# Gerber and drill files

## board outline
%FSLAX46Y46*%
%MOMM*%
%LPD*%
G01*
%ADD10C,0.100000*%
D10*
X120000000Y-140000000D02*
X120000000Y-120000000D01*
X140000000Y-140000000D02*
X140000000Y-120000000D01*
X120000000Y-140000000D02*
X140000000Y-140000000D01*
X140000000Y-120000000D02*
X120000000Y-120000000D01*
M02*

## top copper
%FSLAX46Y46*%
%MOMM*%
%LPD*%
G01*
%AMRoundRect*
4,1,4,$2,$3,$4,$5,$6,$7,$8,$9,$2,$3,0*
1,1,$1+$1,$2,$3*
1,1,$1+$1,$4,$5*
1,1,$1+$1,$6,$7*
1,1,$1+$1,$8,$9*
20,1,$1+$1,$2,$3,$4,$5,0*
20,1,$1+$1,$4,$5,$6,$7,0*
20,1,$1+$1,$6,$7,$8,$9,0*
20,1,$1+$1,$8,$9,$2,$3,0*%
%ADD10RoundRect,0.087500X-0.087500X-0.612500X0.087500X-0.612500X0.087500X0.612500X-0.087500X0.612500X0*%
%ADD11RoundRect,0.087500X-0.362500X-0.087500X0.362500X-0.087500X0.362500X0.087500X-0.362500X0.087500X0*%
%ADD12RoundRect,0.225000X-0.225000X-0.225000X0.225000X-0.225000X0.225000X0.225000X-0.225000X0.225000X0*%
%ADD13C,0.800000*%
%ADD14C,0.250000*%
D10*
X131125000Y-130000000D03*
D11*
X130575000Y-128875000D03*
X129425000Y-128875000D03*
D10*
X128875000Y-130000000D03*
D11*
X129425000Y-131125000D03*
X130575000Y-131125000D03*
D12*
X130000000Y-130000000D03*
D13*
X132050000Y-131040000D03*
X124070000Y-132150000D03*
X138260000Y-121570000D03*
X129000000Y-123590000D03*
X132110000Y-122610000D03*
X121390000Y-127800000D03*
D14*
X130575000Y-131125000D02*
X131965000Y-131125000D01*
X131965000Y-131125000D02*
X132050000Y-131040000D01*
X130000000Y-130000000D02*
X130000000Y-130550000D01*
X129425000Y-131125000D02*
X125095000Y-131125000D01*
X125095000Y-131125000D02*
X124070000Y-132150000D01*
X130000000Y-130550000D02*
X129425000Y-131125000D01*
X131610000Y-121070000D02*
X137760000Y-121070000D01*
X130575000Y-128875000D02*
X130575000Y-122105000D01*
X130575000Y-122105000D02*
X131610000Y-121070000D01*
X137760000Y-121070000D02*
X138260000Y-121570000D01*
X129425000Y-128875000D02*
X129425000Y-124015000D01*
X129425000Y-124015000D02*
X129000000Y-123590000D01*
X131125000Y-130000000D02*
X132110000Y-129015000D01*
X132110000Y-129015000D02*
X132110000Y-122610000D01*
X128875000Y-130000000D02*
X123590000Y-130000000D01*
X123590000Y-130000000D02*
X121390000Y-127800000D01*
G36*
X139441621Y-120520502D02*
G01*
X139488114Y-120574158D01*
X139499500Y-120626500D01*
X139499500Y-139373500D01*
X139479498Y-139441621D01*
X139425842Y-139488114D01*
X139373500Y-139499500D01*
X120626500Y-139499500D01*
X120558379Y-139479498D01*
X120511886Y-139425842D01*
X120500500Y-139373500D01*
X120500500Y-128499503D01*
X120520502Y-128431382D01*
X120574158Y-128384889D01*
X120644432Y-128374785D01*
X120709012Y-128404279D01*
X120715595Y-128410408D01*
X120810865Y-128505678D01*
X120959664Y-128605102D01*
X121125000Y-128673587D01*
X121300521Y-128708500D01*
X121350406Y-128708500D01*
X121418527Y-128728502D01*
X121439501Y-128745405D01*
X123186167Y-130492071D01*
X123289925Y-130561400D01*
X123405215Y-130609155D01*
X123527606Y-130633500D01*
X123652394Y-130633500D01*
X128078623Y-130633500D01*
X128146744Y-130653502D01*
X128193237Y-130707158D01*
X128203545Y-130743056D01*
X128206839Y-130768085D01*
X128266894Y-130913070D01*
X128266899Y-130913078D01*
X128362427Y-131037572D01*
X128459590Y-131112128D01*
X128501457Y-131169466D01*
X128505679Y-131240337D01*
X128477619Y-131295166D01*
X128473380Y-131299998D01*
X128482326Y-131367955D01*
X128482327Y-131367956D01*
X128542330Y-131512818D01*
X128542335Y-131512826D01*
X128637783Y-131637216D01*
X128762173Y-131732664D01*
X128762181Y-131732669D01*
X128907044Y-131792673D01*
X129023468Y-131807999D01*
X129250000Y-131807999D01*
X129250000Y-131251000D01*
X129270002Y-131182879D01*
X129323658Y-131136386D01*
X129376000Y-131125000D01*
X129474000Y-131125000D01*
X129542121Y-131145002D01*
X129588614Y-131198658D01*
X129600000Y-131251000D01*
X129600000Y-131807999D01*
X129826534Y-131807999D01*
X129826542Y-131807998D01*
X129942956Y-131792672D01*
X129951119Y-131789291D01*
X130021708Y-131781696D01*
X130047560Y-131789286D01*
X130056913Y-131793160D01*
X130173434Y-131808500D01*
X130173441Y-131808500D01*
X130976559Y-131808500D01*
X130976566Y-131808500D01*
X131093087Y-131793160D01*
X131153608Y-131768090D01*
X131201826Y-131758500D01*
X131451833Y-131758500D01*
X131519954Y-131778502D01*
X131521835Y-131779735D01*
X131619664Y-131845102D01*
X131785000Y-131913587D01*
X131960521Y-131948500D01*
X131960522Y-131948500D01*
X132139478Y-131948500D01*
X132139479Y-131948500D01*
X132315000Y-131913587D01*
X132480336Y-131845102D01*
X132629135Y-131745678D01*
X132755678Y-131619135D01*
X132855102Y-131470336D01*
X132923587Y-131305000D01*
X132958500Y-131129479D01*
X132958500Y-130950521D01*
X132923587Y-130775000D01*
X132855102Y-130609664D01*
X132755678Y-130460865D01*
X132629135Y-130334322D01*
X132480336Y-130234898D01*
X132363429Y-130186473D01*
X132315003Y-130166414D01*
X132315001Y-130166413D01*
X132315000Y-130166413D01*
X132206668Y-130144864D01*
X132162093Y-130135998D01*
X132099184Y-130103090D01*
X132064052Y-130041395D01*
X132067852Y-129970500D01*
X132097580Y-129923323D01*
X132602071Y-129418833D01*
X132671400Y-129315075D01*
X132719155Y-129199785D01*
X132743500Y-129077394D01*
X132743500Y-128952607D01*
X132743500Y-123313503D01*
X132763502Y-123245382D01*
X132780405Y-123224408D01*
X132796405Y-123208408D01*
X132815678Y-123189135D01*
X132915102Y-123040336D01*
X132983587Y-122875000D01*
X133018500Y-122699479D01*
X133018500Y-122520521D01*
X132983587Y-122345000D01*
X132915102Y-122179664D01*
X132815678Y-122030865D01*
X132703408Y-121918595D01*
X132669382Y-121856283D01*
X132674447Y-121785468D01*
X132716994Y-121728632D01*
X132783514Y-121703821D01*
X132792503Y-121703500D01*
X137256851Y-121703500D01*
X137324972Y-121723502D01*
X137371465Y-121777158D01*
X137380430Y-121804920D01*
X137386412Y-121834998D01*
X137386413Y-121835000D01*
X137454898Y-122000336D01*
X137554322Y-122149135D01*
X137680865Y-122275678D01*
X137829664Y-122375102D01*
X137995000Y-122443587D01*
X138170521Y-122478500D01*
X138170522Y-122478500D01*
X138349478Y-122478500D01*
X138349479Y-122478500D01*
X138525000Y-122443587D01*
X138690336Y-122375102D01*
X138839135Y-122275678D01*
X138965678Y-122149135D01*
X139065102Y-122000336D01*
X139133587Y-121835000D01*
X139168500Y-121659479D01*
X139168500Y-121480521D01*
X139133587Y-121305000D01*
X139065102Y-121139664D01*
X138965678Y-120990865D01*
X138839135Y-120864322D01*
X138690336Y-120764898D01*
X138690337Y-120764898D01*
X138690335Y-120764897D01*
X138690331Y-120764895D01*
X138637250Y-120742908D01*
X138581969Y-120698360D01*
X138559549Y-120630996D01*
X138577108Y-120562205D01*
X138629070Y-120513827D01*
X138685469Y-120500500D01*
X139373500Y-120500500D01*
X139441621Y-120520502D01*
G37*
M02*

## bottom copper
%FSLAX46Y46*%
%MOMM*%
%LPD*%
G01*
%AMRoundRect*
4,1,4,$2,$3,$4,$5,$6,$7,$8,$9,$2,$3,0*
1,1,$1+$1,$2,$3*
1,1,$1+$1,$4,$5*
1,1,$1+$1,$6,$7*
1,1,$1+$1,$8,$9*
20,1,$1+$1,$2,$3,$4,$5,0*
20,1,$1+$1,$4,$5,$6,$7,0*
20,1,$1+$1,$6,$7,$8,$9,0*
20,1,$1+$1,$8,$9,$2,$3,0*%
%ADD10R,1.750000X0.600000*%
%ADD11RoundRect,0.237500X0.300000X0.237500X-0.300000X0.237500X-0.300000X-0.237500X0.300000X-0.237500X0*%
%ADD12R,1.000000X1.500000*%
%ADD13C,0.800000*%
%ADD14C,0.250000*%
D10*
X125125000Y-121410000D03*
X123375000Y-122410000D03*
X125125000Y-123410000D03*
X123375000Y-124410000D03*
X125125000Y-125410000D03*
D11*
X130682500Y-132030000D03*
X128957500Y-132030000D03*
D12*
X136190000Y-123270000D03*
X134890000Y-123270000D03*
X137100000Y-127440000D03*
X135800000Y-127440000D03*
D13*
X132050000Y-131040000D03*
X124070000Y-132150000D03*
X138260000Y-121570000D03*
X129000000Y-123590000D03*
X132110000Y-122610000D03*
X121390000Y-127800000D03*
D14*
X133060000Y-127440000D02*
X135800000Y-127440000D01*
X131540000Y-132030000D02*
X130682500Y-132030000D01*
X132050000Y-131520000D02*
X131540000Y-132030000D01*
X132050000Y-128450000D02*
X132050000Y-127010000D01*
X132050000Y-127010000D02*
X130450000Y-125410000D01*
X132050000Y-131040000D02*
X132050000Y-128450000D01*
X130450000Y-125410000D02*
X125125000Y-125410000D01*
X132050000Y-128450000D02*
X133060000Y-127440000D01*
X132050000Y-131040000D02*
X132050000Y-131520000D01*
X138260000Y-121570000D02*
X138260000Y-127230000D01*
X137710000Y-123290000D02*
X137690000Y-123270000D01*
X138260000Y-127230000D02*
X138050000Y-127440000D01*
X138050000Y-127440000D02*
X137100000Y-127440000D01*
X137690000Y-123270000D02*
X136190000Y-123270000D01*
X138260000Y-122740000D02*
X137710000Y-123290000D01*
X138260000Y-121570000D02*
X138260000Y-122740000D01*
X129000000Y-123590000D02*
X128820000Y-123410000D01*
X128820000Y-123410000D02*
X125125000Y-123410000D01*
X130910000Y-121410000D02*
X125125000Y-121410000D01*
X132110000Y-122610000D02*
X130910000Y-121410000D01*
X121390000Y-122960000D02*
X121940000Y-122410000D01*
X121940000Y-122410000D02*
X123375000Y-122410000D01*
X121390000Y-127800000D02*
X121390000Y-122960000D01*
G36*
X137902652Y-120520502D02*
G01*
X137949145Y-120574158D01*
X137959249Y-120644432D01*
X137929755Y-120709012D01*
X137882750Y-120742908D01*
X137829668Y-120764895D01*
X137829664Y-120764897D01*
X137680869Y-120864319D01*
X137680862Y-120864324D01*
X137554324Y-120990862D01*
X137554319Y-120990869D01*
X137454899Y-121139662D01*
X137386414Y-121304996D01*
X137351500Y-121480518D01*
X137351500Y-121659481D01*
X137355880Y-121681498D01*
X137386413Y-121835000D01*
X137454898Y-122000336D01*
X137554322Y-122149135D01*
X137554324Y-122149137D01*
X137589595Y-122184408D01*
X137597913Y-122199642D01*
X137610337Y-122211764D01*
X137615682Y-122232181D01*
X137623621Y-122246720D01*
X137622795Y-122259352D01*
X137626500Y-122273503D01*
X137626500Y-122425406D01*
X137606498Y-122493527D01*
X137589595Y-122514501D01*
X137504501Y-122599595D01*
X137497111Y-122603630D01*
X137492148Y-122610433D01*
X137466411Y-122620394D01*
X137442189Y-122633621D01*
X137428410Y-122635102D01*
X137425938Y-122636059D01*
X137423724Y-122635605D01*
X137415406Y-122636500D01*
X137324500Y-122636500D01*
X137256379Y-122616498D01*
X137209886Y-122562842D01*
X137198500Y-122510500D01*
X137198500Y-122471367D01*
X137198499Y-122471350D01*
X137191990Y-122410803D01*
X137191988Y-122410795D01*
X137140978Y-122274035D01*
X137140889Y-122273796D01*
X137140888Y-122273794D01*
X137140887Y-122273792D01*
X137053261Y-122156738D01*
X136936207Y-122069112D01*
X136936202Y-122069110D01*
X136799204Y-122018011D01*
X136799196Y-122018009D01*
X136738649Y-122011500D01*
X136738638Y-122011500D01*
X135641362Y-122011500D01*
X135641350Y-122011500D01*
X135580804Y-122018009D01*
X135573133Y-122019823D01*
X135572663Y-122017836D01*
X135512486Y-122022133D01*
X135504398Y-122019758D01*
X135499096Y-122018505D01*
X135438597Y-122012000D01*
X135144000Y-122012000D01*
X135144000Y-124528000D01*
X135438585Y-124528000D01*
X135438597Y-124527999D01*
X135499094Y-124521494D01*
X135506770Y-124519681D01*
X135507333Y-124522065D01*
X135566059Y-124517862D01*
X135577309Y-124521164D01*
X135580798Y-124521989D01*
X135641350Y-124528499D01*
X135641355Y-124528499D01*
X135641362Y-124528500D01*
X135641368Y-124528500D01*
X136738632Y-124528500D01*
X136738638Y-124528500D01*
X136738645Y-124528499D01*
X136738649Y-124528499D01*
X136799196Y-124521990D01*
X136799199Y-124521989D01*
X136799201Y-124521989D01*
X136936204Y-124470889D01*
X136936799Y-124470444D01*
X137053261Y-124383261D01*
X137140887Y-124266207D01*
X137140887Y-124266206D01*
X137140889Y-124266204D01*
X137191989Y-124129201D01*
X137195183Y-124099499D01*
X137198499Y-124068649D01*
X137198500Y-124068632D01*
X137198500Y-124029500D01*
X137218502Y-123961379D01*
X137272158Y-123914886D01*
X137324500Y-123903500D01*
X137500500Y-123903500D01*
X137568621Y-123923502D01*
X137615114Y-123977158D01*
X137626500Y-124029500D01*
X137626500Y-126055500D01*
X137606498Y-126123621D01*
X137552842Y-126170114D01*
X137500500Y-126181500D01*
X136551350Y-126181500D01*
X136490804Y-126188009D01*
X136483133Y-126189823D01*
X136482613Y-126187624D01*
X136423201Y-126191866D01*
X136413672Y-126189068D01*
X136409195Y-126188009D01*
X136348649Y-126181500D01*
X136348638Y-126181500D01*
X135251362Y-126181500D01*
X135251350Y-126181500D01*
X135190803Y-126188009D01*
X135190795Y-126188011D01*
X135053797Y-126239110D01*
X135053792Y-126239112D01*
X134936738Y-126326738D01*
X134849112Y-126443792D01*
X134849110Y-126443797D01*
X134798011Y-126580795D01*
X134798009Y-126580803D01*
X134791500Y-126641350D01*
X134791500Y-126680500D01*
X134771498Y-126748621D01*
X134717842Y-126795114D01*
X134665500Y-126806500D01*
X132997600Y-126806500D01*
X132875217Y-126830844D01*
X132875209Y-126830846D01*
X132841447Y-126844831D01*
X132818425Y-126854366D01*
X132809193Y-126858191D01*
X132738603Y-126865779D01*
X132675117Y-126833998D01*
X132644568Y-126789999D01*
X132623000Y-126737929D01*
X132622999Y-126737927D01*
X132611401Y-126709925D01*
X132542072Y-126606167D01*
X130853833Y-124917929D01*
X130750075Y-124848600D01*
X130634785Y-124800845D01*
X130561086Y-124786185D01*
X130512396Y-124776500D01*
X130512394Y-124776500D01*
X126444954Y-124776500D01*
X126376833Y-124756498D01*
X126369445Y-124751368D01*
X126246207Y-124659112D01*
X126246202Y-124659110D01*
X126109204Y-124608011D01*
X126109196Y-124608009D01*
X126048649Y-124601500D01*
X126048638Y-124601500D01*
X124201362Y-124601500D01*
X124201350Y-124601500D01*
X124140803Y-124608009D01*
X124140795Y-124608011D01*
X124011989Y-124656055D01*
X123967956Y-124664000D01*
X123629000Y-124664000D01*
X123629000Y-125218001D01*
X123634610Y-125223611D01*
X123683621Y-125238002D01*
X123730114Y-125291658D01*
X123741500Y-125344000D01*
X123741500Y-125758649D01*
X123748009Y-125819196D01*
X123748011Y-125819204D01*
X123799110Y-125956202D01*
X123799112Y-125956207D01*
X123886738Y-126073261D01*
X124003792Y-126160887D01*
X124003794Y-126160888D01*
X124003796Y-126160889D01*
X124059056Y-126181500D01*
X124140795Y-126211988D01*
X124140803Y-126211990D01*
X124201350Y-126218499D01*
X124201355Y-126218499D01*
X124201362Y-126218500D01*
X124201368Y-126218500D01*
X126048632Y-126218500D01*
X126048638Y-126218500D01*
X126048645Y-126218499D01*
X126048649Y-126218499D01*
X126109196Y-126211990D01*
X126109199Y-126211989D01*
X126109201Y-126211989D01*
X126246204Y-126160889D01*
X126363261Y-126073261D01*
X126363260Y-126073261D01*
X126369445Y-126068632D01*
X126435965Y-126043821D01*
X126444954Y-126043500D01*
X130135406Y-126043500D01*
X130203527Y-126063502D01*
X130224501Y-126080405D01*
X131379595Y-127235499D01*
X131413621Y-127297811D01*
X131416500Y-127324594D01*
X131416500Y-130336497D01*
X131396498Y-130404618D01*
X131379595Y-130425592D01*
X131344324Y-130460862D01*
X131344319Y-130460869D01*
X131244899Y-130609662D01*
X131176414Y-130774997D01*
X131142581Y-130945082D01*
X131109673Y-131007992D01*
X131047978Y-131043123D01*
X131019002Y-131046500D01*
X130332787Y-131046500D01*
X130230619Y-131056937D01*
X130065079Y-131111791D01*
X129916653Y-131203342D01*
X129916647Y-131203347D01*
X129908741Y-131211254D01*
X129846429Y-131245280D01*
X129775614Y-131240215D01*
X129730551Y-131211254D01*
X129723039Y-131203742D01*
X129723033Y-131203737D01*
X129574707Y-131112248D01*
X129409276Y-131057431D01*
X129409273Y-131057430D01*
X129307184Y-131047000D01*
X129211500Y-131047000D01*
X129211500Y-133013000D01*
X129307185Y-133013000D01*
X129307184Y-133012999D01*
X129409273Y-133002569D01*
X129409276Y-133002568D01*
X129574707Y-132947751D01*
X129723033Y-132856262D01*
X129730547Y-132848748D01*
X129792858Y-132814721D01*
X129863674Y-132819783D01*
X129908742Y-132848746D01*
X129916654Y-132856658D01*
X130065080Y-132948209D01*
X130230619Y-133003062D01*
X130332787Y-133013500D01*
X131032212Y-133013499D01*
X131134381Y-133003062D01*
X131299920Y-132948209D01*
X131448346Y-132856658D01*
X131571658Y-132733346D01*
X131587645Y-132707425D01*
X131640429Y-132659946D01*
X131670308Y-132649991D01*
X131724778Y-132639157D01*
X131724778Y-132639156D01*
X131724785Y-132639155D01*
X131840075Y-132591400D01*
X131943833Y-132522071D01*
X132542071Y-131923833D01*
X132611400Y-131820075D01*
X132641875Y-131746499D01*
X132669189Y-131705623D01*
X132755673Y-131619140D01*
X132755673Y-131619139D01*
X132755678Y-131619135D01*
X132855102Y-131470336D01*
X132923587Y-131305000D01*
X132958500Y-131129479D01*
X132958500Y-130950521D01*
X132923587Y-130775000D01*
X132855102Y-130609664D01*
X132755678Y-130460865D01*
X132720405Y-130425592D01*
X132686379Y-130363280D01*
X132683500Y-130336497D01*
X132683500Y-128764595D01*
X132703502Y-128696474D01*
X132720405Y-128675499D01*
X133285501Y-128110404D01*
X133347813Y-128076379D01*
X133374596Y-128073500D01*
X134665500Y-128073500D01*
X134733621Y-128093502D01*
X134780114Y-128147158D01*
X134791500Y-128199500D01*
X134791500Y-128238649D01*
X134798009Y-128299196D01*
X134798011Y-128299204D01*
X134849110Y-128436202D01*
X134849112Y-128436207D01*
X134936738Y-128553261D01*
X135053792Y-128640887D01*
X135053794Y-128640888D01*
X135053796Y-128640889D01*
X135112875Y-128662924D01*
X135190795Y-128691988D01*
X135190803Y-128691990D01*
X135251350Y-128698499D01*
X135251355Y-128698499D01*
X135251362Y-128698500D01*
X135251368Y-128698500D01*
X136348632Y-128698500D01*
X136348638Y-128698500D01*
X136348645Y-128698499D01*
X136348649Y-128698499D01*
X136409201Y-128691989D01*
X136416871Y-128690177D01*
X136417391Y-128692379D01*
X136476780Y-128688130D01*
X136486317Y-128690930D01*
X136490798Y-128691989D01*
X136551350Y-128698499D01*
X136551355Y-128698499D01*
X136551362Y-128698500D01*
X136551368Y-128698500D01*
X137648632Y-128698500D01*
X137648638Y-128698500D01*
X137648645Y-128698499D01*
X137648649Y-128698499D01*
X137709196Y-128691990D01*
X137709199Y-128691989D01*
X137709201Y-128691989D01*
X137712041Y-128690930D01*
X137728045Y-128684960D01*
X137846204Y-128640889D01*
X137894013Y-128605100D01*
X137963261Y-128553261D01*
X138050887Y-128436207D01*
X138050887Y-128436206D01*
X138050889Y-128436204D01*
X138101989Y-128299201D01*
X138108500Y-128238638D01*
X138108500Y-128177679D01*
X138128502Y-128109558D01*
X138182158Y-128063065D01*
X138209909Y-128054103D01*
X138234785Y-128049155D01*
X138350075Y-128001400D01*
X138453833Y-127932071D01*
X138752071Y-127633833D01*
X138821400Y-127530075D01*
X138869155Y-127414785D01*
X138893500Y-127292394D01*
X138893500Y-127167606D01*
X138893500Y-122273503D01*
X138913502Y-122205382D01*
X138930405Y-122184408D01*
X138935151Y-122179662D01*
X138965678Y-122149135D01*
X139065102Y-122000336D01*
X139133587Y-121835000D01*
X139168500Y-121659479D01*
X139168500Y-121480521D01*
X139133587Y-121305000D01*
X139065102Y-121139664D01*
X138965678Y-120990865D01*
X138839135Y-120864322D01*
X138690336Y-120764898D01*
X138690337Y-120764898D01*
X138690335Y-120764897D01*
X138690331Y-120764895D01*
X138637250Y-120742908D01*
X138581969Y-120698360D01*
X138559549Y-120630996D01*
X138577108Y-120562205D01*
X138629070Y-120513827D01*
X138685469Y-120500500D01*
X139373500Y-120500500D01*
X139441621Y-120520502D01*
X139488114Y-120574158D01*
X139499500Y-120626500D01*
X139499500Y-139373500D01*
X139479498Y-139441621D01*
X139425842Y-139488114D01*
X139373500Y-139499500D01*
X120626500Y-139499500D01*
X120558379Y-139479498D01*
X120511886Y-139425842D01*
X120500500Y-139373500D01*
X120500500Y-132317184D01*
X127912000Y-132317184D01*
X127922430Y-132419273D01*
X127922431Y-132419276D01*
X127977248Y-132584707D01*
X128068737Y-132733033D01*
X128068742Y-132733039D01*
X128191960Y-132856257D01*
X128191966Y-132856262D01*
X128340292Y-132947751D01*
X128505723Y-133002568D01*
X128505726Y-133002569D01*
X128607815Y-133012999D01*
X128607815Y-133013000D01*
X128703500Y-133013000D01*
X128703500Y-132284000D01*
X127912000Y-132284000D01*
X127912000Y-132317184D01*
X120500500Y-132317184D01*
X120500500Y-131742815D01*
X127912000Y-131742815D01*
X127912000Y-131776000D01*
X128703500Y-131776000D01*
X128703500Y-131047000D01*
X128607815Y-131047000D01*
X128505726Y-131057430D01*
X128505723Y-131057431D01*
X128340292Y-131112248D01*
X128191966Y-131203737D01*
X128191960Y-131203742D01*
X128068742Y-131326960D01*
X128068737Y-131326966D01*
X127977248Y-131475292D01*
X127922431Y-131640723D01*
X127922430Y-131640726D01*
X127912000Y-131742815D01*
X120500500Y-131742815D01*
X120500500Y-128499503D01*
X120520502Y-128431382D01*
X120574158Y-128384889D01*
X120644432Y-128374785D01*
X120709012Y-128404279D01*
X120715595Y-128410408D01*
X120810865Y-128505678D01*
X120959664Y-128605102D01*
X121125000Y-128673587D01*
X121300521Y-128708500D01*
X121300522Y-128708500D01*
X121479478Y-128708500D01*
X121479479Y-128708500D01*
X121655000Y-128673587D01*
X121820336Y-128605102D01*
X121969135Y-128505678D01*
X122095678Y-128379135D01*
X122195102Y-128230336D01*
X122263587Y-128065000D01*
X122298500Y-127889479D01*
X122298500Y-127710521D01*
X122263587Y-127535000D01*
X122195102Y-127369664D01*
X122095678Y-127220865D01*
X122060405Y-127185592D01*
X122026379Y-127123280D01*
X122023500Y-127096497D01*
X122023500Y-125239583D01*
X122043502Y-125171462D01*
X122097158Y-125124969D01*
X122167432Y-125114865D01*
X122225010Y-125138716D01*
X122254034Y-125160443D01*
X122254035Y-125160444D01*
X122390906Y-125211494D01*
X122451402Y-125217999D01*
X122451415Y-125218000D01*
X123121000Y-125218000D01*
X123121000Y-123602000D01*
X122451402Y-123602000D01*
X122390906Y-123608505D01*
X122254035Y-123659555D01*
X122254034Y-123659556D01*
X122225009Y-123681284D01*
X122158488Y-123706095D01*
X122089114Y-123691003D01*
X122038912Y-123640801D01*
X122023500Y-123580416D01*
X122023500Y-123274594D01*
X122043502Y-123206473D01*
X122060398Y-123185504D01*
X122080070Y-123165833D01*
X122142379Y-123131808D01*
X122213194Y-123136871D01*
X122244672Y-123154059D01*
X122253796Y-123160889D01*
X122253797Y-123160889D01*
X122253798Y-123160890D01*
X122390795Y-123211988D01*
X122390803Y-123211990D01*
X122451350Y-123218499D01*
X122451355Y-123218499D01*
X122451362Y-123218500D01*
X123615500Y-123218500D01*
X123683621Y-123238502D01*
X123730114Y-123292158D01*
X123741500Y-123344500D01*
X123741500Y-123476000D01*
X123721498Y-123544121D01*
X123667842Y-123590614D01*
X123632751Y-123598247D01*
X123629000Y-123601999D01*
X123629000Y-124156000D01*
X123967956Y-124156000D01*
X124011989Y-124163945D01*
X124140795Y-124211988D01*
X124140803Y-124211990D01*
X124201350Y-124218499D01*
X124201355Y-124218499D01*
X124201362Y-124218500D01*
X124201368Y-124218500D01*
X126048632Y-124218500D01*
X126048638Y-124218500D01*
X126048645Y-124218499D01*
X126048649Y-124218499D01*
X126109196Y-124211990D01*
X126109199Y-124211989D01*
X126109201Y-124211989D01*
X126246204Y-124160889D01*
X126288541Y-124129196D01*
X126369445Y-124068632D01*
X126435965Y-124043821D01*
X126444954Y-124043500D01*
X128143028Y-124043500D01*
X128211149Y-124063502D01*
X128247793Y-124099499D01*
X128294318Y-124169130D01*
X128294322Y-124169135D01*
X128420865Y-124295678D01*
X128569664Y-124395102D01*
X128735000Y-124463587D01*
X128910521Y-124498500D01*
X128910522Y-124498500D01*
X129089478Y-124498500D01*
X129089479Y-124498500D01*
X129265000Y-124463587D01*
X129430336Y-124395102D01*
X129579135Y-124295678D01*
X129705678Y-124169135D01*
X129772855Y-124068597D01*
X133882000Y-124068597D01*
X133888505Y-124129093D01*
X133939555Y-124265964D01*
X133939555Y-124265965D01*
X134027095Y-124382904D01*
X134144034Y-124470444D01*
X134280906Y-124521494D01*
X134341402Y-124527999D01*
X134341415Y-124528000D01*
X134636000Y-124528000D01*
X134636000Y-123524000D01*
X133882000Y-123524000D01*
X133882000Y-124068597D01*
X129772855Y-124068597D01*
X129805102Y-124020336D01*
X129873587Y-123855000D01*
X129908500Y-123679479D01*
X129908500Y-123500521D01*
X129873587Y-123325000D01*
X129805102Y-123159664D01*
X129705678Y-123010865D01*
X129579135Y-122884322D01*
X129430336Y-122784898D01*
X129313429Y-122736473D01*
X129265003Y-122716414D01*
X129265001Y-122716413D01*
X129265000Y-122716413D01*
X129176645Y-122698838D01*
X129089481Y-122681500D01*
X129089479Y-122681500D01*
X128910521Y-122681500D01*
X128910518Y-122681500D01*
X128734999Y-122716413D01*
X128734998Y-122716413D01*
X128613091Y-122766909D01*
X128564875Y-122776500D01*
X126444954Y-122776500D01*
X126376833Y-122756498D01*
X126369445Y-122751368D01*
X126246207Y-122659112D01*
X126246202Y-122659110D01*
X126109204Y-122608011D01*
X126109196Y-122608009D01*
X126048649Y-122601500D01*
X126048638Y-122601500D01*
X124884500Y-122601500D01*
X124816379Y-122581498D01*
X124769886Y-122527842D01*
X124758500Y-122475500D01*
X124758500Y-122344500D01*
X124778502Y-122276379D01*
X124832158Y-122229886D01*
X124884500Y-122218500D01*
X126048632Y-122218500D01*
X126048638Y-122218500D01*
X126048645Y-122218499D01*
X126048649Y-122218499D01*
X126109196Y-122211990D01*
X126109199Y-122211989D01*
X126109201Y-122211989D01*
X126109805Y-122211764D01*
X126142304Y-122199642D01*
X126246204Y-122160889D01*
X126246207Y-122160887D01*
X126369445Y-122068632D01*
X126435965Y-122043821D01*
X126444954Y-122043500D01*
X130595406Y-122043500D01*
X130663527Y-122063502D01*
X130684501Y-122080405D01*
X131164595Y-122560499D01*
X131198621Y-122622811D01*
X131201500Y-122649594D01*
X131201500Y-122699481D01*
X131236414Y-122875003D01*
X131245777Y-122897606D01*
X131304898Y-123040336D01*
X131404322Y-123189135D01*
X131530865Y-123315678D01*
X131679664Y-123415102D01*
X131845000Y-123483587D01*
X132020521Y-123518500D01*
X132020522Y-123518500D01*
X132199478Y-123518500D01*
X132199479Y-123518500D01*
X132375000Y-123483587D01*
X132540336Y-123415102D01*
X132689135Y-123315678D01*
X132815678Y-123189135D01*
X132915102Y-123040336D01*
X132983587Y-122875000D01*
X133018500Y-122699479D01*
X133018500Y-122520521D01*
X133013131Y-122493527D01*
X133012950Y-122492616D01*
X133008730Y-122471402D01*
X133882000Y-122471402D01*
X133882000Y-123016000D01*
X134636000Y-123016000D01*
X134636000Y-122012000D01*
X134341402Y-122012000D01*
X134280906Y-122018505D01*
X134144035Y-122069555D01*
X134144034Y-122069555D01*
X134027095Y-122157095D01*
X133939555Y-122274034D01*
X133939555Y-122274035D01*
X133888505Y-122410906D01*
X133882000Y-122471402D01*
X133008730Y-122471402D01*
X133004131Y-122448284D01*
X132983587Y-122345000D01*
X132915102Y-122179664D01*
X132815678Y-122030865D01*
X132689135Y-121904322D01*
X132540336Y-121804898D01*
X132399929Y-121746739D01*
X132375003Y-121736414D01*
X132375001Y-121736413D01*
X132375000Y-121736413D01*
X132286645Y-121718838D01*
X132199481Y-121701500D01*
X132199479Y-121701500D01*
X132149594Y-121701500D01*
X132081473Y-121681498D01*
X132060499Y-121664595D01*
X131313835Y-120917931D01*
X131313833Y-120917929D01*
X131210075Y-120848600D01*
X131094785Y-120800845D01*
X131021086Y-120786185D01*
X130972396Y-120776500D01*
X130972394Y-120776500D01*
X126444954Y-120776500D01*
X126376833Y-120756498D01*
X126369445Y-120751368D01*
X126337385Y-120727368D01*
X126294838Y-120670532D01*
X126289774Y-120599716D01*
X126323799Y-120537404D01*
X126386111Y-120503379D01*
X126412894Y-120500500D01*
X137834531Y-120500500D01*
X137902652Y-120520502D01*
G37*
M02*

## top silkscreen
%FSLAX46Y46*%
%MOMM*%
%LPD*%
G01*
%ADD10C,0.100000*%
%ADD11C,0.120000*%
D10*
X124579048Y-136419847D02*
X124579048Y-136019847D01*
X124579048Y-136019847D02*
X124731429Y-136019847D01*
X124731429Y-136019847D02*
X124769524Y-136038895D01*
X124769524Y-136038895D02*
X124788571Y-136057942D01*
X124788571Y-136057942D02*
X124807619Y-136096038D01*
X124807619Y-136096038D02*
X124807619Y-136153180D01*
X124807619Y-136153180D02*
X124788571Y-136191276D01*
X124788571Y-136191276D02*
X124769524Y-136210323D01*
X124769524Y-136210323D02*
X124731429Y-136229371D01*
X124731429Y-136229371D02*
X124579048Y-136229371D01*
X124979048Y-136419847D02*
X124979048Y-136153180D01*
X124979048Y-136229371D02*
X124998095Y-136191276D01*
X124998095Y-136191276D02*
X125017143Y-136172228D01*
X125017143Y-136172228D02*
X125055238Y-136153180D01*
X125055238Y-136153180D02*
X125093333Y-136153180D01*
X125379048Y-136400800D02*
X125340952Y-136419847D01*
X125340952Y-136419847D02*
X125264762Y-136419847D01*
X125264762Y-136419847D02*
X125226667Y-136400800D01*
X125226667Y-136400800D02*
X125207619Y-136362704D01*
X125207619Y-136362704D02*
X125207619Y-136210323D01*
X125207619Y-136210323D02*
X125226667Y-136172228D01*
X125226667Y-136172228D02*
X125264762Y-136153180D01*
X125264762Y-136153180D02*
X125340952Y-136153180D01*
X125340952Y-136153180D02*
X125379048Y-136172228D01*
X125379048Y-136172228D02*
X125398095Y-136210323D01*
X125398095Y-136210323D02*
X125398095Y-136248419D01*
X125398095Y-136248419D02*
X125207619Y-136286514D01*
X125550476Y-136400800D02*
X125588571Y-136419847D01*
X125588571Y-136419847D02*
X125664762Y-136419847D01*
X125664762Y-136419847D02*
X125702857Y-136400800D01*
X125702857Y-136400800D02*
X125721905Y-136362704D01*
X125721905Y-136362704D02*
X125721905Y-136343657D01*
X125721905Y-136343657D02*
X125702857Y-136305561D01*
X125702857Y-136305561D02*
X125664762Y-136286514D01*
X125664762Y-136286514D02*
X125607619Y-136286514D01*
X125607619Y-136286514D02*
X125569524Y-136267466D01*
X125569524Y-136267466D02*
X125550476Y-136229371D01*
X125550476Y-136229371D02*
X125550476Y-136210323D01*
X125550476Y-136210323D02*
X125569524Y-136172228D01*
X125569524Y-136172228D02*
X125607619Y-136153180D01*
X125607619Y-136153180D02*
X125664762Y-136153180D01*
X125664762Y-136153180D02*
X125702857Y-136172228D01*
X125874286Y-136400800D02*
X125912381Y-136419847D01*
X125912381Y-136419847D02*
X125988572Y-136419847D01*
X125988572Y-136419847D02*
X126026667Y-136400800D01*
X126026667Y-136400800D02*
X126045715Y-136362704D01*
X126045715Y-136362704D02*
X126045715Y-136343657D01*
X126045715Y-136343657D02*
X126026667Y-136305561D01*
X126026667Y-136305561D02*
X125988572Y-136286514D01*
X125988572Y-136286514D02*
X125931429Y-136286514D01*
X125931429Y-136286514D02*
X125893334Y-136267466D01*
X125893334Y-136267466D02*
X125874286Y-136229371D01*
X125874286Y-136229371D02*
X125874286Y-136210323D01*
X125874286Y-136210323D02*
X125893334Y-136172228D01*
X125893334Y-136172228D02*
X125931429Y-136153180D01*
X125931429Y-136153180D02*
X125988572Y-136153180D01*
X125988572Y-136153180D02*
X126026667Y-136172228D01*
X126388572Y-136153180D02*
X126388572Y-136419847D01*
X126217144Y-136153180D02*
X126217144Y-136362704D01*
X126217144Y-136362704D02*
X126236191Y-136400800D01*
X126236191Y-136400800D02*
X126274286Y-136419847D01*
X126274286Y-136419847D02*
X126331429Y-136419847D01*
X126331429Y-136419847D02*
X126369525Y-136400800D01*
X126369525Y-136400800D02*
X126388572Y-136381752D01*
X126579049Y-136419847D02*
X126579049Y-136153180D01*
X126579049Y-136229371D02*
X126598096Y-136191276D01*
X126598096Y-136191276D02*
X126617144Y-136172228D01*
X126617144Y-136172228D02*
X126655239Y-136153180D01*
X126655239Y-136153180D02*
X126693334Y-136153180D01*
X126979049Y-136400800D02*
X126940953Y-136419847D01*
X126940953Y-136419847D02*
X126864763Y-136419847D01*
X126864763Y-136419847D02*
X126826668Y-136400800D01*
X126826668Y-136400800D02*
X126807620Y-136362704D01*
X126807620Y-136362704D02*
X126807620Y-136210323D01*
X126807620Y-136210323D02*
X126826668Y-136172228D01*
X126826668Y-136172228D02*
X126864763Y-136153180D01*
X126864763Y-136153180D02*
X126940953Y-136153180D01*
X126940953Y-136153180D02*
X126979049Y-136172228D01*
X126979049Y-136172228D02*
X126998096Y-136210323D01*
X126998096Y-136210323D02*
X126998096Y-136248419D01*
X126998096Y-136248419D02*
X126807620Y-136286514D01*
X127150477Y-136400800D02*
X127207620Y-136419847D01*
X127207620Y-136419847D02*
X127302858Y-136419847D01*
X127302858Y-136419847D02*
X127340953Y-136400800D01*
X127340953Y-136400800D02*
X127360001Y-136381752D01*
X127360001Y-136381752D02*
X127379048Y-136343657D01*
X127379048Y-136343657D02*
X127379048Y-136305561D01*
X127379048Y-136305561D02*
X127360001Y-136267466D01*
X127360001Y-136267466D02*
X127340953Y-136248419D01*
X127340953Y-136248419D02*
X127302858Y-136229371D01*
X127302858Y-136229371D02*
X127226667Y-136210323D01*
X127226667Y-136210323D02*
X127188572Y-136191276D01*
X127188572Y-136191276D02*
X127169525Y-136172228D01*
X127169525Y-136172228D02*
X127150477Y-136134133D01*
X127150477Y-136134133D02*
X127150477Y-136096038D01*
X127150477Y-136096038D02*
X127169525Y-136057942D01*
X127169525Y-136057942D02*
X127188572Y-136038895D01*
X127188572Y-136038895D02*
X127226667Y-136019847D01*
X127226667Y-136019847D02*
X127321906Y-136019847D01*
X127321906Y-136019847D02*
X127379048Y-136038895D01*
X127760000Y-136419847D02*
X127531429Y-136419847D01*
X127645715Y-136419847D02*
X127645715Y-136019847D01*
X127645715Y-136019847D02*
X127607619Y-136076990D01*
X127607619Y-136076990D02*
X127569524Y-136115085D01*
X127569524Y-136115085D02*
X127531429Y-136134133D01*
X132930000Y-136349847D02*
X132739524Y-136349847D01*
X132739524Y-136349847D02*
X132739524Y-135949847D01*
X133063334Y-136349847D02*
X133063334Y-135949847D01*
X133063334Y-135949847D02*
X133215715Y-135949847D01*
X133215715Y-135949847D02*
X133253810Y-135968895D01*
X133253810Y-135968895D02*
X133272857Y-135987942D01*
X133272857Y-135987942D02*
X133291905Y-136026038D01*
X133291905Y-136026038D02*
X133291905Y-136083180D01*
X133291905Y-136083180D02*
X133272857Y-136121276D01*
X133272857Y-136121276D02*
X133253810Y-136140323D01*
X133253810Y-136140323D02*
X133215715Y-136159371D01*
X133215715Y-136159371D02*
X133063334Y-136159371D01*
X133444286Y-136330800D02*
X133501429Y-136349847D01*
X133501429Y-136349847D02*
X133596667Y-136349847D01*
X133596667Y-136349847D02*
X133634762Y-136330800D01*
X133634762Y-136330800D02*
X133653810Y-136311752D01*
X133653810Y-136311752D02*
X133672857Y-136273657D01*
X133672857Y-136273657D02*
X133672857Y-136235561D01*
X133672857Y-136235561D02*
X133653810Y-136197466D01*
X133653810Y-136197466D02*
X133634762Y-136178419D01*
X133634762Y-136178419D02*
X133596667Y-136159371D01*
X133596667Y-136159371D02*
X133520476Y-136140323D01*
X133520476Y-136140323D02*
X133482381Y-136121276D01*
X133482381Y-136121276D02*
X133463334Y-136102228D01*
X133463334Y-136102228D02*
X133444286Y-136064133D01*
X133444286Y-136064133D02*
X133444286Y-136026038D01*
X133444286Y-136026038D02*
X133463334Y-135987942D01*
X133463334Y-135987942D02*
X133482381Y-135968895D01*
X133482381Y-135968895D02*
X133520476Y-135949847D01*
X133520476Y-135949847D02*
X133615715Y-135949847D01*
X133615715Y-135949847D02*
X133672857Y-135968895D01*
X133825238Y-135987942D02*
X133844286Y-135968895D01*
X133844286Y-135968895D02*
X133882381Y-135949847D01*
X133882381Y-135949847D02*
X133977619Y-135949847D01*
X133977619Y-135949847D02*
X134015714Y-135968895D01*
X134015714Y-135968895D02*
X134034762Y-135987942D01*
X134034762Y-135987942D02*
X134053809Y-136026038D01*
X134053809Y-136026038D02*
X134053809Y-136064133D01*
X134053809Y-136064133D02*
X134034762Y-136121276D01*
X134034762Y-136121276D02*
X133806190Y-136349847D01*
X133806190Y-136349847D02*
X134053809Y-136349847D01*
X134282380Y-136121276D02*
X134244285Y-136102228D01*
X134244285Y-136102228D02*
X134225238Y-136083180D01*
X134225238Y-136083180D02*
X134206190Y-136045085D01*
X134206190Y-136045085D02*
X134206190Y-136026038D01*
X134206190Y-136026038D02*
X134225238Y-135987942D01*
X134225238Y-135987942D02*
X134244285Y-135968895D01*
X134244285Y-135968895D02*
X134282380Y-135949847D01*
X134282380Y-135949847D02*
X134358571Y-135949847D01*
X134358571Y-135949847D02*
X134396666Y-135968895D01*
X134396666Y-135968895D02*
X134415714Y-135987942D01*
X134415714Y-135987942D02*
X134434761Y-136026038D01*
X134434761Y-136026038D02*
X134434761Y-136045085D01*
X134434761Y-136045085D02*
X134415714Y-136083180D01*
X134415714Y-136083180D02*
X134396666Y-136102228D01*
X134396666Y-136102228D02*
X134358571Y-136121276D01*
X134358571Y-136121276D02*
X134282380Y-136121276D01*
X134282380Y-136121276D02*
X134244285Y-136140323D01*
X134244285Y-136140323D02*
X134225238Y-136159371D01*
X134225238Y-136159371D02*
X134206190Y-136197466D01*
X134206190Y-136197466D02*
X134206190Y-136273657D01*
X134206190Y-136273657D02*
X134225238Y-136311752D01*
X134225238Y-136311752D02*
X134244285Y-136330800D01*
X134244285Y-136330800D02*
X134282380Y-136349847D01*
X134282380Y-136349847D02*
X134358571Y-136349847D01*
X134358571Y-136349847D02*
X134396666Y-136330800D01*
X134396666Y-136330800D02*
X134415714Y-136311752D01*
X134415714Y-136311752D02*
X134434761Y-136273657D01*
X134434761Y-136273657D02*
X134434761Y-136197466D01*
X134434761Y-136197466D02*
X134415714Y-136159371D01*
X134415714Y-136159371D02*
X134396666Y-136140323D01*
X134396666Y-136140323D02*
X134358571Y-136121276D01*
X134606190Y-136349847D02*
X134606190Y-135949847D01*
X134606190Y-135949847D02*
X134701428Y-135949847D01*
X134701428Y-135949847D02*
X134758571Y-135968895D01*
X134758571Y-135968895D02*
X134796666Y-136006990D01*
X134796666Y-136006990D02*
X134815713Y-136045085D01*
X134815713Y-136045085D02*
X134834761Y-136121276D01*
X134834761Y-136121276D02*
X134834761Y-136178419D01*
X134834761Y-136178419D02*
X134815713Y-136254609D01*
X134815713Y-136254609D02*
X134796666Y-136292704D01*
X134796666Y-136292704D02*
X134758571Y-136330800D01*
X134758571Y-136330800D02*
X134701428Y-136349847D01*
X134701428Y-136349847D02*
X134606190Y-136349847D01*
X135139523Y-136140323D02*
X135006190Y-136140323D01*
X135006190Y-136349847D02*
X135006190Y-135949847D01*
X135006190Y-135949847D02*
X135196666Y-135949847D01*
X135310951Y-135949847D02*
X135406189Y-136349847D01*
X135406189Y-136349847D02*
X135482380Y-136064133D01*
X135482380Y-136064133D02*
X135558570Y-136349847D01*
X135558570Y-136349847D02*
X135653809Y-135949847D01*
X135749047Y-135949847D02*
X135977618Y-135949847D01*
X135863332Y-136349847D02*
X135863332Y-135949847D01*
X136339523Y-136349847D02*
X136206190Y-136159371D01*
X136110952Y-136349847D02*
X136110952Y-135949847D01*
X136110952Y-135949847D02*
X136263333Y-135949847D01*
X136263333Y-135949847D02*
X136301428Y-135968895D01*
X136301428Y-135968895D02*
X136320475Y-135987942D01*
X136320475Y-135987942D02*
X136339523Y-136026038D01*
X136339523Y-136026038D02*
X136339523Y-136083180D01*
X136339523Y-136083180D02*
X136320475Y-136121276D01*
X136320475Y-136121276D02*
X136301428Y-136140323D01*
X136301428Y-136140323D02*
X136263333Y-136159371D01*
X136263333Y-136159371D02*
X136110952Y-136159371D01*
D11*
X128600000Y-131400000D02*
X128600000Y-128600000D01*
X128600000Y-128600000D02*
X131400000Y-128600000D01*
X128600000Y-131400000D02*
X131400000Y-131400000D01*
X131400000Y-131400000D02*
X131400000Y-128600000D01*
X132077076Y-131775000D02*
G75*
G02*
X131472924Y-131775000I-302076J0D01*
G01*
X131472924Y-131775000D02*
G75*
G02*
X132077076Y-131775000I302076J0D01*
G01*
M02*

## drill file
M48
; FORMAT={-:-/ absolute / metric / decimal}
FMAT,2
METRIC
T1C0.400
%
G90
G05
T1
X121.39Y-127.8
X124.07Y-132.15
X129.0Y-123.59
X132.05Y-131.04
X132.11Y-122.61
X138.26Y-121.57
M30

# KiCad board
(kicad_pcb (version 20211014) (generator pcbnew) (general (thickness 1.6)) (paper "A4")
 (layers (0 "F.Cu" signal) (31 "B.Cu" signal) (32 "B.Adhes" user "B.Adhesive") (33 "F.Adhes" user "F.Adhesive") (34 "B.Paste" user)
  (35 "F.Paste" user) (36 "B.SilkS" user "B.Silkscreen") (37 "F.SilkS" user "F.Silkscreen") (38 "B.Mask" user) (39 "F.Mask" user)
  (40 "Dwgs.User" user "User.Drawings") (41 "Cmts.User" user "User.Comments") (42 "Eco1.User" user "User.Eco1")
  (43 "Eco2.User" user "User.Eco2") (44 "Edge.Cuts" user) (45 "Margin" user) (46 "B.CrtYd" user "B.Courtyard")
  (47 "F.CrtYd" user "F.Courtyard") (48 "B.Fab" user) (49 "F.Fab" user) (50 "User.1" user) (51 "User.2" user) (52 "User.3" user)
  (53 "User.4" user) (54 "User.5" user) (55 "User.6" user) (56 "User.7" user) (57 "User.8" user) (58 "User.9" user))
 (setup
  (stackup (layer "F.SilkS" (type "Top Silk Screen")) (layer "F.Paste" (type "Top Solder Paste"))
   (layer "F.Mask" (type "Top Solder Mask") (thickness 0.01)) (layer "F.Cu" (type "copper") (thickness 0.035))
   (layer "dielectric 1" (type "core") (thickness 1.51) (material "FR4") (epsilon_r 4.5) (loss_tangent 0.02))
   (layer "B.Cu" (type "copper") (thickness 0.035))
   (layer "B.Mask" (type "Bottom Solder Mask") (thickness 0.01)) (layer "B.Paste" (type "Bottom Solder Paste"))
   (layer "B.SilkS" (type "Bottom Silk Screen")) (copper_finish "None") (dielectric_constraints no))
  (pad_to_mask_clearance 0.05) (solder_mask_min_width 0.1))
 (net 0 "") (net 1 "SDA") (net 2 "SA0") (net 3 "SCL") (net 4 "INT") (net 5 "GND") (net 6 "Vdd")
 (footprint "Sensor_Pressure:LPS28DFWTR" (layer "F.Cu") (at 130 130)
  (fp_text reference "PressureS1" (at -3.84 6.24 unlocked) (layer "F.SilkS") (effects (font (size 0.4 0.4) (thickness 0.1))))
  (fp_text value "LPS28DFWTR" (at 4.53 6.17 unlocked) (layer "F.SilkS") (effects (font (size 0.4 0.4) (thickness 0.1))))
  (fp_line (start -1.4 1.4) (end -1.4 -1.4) (layer "F.SilkS") (width 0.12))
  (fp_line (start -1.4 -1.4) (end 1.4 -1.4) (layer "F.SilkS") (width 0.12))
  (fp_line (start -1.4 1.4) (end 1.4 1.4) (layer "F.SilkS") (width 0.12))
  (fp_line (start 1.4 1.4) (end 1.4 -1.4) (layer "F.SilkS") (width 0.12))
  (fp_circle (center 1.775 1.775) (end 2.05 1.9) (layer "F.SilkS") (width 0.12) (fill none))
  (pad "1" smd roundrect (at 1.125 0) (size 0.35 1.4) (layers "F.Cu" "F.Paste" "F.Mask") (roundrect_rratio 0.25) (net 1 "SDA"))
  (pad "2" smd roundrect (at 0.575 -1.125) (size 0.9 0.35) (layers "F.Cu" "F.Paste" "F.Mask") (roundrect_rratio 0.25) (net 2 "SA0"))
  (pad "3" smd roundrect (at -0.575 -1.125) (size 0.9 0.35) (layers "F.Cu" "F.Paste" "F.Mask") (roundrect_rratio 0.25) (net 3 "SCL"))
  (pad "4" smd roundrect (at -1.125 0) (size 0.35 1.4) (layers "F.Cu" "F.Paste" "F.Mask") (roundrect_rratio 0.25) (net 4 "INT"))
  (pad "5" smd roundrect (at -0.575 1.125) (size 0.9 0.35) (layers "F.Cu" "F.Paste" "F.Mask") (roundrect_rratio 0.25) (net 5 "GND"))
  (pad "6" smd roundrect (at 0.575 1.125) (size 0.9 0.35) (layers "F.Cu" "F.Paste" "F.Mask") (roundrect_rratio 0.25) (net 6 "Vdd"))
  (pad "7" smd roundrect (at 0 0) (size 0.9 0.9) (layers "F.Cu" "F.Paste" "F.Mask") (roundrect_rratio 0.25) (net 5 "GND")))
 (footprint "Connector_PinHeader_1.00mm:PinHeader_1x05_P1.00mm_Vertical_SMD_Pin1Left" (layer "B.Cu") (at 124.25 123.41 180)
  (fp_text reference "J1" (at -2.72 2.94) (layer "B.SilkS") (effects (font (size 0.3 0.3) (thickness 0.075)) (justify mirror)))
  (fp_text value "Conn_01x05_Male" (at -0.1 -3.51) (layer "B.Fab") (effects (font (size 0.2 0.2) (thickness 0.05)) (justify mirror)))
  (pad "1" smd rect (at -0.875 2 180) (size 1.75 0.6) (layers "B.Cu" "B.Paste" "B.Mask") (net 1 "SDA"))
  (pad "2" smd rect (at 0.875 1 180) (size 1.75 0.6) (layers "B.Cu" "B.Paste" "B.Mask") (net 4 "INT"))
  (pad "3" smd rect (at -0.875 0 180) (size 1.75 0.6) (layers "B.Cu" "B.Paste" "B.Mask") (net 3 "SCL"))
  (pad "4" smd rect (at 0.875 -1 180) (size 1.75 0.6) (layers "B.Cu" "B.Paste" "B.Mask") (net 5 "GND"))
  (pad "5" smd rect (at -0.875 -2 180) (size 1.75 0.6) (layers "B.Cu" "B.Paste" "B.Mask") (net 6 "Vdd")))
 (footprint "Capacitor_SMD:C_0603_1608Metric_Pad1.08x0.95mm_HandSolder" (layer "B.Cu") (at 129.82 132.03 180)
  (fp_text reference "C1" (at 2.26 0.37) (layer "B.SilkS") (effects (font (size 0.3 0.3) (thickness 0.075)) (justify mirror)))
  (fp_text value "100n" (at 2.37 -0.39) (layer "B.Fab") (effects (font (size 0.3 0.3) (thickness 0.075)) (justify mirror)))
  (pad "1" smd roundrect (at -0.8625 0 180) (size 1.075 0.95) (layers "B.Cu" "B.Paste" "B.Mask") (roundrect_rratio 0.25) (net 6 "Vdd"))
  (pad "2" smd roundrect (at 0.8625 0 180) (size 1.075 0.95) (layers "B.Cu" "B.Paste" "B.Mask") (roundrect_rratio 0.25) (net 5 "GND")))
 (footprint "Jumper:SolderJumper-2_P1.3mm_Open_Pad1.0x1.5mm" (layer "B.Cu") (at 135.54 123.27 180)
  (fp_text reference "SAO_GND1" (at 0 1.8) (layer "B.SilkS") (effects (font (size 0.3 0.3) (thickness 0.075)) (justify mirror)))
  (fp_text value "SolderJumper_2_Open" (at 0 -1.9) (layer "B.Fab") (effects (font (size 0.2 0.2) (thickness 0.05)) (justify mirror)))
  (pad "1" smd rect (at -0.65 0 180) (size 1 1.5) (layers "B.Cu" "B.Mask") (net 2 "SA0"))
  (pad "2" smd rect (at 0.65 0 180) (size 1 1.5) (layers "B.Cu" "B.Mask") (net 5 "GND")))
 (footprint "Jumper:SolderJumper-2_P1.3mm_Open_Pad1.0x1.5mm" (layer "B.Cu") (at 136.45 127.44 180)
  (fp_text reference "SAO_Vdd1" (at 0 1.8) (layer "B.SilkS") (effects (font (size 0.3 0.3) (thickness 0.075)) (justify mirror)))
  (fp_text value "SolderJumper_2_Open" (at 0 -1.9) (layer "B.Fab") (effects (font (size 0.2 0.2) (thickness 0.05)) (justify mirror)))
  (pad "1" smd rect (at -0.65 0 180) (size 1 1.5) (layers "B.Cu" "B.Mask") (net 2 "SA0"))
  (pad "2" smd rect (at 0.65 0 180) (size 1 1.5) (layers "B.Cu" "B.Mask") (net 6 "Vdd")))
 (gr_line (start 120 140) (end 120 120) (layer "Edge.Cuts") (width 0.1))
 (gr_line (start 140 140) (end 140 120) (layer "Edge.Cuts") (width 0.1))
 (gr_line (start 120 140) (end 140 140) (layer "Edge.Cuts") (width 0.1))
 (gr_line (start 140 120) (end 120 120) (layer "Edge.Cuts") (width 0.1))
 (segment (start 130.575 131.125) (end 131.965 131.125) (width 0.25) (layer "F.Cu") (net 6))
 (segment (start 131.965 131.125) (end 132.05 131.04) (width 0.25) (layer "F.Cu") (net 6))
 (via (at 132.05 131.04) (size 0.8) (drill 0.4) (layers "F.Cu" "B.Cu") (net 6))
 (segment (start 133.06 127.44) (end 135.8 127.44) (width 0.25) (layer "B.Cu") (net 6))
 (segment (start 131.54 132.03) (end 130.6825 132.03) (width 0.25) (layer "B.Cu") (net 6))
 (segment (start 132.05 131.52) (end 131.54 132.03) (width 0.25) (layer "B.Cu") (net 6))
 (segment (start 132.05 128.45) (end 132.05 127.01) (width 0.25) (layer "B.Cu") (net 6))
 (segment (start 132.05 127.01) (end 130.45 125.41) (width 0.25) (layer "B.Cu") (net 6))
 (segment (start 132.05 131.04) (end 132.05 128.45) (width 0.25) (layer "B.Cu") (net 6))
 (segment (start 130.45 125.41) (end 125.125 125.41) (width 0.25) (layer "B.Cu") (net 6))
 (segment (start 132.05 128.45) (end 133.06 127.44) (width 0.25) (layer "B.Cu") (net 6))
 (segment (start 132.05 131.04) (end 132.05 131.52) (width 0.25) (layer "B.Cu") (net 6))
 (segment (start 130 130) (end 130 130.55) (width 0.25) (layer "F.Cu") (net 5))
 (segment (start 129.425 131.125) (end 125.095 131.125) (width 0.25) (layer "F.Cu") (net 5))
 (segment (start 125.095 131.125) (end 124.07 132.15) (width 0.25) (layer "F.Cu") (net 5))
 (segment (start 130 130.55) (end 129.425 131.125) (width 0.25) (layer "F.Cu") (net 5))
 (via (at 124.07 132.15) (size 0.8) (drill 0.4) (layers "F.Cu" "B.Cu") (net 5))
 (segment (start 131.61 121.07) (end 137.76 121.07) (width 0.25) (layer "F.Cu") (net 2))
 (segment (start 130.575 128.875) (end 130.575 122.105) (width 0.25) (layer "F.Cu") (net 2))
 (segment (start 130.575 122.105) (end 131.61 121.07) (width 0.25) (layer "F.Cu") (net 2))
 (segment (start 137.76 121.07) (end 138.26 121.57) (width 0.25) (layer "F.Cu") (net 2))
 (via (at 138.26 121.57) (size 0.8) (drill 0.4) (layers "F.Cu" "B.Cu") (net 2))
 (segment (start 138.26 121.57) (end 138.26 127.23) (width 0.25) (layer "B.Cu") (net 2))
 (segment (start 137.71 123.29) (end 137.69 123.27) (width 0.25) (layer "B.Cu") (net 2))
 (segment (start 138.26 127.23) (end 138.05 127.44) (width 0.25) (layer "B.Cu") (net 2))
 (segment (start 138.05 127.44) (end 137.1 127.44) (width 0.25) (layer "B.Cu") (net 2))
 (segment (start 137.69 123.27) (end 136.19 123.27) (width 0.25) (layer "B.Cu") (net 2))
 (segment (start 138.26 122.74) (end 137.71 123.29) (width 0.25) (layer "B.Cu") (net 2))
 (segment (start 138.26 121.57) (end 138.26 122.74) (width 0.25) (layer "B.Cu") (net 2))
 (segment (start 129.425 128.875) (end 129.425 124.015) (width 0.25) (layer "F.Cu") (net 3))
 (segment (start 129.425 124.015) (end 129 123.59) (width 0.25) (layer "F.Cu") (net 3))
 (via (at 129 123.59) (size 0.8) (drill 0.4) (layers "F.Cu" "B.Cu") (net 3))
 (segment (start 129 123.59) (end 128.82 123.41) (width 0.25) (layer "B.Cu") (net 3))
 (segment (start 128.82 123.41) (end 125.125 123.41) (width 0.25) (layer "B.Cu") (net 3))
 (segment (start 131.125 130) (end 132.11 129.015) (width 0.25) (layer "F.Cu") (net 1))
 (segment (start 132.11 129.015) (end 132.11 122.61) (width 0.25) (layer "F.Cu") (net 1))
 (via (at 132.11 122.61) (size 0.8) (drill 0.4) (layers "F.Cu" "B.Cu") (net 1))
 (segment (start 130.91 121.41) (end 125.125 121.41) (width 0.25) (layer "B.Cu") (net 1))
 (segment (start 132.11 122.61) (end 130.91 121.41) (width 0.25) (layer "B.Cu") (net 1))
 (segment (start 128.875 130) (end 123.59 130) (width 0.25) (layer "F.Cu") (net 4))
 (segment (start 123.59 130) (end 121.39 127.8) (width 0.25) (layer "F.Cu") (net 4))
 (via (at 121.39 127.8) (size 0.8) (drill 0.4) (layers "F.Cu" "B.Cu") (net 4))
 (segment (start 121.39 122.96) (end 121.94 122.41) (width 0.25) (layer "B.Cu") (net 4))
 (segment (start 121.94 122.41) (end 123.375 122.41) (width 0.25) (layer "B.Cu") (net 4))
 (segment (start 121.39 127.8) (end 121.39 122.96) (width 0.25) (layer "B.Cu") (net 4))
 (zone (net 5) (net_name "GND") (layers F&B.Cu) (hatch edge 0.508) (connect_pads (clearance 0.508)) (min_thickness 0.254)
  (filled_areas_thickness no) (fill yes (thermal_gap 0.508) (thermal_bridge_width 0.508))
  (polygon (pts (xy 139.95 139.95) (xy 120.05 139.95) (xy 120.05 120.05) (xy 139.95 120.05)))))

